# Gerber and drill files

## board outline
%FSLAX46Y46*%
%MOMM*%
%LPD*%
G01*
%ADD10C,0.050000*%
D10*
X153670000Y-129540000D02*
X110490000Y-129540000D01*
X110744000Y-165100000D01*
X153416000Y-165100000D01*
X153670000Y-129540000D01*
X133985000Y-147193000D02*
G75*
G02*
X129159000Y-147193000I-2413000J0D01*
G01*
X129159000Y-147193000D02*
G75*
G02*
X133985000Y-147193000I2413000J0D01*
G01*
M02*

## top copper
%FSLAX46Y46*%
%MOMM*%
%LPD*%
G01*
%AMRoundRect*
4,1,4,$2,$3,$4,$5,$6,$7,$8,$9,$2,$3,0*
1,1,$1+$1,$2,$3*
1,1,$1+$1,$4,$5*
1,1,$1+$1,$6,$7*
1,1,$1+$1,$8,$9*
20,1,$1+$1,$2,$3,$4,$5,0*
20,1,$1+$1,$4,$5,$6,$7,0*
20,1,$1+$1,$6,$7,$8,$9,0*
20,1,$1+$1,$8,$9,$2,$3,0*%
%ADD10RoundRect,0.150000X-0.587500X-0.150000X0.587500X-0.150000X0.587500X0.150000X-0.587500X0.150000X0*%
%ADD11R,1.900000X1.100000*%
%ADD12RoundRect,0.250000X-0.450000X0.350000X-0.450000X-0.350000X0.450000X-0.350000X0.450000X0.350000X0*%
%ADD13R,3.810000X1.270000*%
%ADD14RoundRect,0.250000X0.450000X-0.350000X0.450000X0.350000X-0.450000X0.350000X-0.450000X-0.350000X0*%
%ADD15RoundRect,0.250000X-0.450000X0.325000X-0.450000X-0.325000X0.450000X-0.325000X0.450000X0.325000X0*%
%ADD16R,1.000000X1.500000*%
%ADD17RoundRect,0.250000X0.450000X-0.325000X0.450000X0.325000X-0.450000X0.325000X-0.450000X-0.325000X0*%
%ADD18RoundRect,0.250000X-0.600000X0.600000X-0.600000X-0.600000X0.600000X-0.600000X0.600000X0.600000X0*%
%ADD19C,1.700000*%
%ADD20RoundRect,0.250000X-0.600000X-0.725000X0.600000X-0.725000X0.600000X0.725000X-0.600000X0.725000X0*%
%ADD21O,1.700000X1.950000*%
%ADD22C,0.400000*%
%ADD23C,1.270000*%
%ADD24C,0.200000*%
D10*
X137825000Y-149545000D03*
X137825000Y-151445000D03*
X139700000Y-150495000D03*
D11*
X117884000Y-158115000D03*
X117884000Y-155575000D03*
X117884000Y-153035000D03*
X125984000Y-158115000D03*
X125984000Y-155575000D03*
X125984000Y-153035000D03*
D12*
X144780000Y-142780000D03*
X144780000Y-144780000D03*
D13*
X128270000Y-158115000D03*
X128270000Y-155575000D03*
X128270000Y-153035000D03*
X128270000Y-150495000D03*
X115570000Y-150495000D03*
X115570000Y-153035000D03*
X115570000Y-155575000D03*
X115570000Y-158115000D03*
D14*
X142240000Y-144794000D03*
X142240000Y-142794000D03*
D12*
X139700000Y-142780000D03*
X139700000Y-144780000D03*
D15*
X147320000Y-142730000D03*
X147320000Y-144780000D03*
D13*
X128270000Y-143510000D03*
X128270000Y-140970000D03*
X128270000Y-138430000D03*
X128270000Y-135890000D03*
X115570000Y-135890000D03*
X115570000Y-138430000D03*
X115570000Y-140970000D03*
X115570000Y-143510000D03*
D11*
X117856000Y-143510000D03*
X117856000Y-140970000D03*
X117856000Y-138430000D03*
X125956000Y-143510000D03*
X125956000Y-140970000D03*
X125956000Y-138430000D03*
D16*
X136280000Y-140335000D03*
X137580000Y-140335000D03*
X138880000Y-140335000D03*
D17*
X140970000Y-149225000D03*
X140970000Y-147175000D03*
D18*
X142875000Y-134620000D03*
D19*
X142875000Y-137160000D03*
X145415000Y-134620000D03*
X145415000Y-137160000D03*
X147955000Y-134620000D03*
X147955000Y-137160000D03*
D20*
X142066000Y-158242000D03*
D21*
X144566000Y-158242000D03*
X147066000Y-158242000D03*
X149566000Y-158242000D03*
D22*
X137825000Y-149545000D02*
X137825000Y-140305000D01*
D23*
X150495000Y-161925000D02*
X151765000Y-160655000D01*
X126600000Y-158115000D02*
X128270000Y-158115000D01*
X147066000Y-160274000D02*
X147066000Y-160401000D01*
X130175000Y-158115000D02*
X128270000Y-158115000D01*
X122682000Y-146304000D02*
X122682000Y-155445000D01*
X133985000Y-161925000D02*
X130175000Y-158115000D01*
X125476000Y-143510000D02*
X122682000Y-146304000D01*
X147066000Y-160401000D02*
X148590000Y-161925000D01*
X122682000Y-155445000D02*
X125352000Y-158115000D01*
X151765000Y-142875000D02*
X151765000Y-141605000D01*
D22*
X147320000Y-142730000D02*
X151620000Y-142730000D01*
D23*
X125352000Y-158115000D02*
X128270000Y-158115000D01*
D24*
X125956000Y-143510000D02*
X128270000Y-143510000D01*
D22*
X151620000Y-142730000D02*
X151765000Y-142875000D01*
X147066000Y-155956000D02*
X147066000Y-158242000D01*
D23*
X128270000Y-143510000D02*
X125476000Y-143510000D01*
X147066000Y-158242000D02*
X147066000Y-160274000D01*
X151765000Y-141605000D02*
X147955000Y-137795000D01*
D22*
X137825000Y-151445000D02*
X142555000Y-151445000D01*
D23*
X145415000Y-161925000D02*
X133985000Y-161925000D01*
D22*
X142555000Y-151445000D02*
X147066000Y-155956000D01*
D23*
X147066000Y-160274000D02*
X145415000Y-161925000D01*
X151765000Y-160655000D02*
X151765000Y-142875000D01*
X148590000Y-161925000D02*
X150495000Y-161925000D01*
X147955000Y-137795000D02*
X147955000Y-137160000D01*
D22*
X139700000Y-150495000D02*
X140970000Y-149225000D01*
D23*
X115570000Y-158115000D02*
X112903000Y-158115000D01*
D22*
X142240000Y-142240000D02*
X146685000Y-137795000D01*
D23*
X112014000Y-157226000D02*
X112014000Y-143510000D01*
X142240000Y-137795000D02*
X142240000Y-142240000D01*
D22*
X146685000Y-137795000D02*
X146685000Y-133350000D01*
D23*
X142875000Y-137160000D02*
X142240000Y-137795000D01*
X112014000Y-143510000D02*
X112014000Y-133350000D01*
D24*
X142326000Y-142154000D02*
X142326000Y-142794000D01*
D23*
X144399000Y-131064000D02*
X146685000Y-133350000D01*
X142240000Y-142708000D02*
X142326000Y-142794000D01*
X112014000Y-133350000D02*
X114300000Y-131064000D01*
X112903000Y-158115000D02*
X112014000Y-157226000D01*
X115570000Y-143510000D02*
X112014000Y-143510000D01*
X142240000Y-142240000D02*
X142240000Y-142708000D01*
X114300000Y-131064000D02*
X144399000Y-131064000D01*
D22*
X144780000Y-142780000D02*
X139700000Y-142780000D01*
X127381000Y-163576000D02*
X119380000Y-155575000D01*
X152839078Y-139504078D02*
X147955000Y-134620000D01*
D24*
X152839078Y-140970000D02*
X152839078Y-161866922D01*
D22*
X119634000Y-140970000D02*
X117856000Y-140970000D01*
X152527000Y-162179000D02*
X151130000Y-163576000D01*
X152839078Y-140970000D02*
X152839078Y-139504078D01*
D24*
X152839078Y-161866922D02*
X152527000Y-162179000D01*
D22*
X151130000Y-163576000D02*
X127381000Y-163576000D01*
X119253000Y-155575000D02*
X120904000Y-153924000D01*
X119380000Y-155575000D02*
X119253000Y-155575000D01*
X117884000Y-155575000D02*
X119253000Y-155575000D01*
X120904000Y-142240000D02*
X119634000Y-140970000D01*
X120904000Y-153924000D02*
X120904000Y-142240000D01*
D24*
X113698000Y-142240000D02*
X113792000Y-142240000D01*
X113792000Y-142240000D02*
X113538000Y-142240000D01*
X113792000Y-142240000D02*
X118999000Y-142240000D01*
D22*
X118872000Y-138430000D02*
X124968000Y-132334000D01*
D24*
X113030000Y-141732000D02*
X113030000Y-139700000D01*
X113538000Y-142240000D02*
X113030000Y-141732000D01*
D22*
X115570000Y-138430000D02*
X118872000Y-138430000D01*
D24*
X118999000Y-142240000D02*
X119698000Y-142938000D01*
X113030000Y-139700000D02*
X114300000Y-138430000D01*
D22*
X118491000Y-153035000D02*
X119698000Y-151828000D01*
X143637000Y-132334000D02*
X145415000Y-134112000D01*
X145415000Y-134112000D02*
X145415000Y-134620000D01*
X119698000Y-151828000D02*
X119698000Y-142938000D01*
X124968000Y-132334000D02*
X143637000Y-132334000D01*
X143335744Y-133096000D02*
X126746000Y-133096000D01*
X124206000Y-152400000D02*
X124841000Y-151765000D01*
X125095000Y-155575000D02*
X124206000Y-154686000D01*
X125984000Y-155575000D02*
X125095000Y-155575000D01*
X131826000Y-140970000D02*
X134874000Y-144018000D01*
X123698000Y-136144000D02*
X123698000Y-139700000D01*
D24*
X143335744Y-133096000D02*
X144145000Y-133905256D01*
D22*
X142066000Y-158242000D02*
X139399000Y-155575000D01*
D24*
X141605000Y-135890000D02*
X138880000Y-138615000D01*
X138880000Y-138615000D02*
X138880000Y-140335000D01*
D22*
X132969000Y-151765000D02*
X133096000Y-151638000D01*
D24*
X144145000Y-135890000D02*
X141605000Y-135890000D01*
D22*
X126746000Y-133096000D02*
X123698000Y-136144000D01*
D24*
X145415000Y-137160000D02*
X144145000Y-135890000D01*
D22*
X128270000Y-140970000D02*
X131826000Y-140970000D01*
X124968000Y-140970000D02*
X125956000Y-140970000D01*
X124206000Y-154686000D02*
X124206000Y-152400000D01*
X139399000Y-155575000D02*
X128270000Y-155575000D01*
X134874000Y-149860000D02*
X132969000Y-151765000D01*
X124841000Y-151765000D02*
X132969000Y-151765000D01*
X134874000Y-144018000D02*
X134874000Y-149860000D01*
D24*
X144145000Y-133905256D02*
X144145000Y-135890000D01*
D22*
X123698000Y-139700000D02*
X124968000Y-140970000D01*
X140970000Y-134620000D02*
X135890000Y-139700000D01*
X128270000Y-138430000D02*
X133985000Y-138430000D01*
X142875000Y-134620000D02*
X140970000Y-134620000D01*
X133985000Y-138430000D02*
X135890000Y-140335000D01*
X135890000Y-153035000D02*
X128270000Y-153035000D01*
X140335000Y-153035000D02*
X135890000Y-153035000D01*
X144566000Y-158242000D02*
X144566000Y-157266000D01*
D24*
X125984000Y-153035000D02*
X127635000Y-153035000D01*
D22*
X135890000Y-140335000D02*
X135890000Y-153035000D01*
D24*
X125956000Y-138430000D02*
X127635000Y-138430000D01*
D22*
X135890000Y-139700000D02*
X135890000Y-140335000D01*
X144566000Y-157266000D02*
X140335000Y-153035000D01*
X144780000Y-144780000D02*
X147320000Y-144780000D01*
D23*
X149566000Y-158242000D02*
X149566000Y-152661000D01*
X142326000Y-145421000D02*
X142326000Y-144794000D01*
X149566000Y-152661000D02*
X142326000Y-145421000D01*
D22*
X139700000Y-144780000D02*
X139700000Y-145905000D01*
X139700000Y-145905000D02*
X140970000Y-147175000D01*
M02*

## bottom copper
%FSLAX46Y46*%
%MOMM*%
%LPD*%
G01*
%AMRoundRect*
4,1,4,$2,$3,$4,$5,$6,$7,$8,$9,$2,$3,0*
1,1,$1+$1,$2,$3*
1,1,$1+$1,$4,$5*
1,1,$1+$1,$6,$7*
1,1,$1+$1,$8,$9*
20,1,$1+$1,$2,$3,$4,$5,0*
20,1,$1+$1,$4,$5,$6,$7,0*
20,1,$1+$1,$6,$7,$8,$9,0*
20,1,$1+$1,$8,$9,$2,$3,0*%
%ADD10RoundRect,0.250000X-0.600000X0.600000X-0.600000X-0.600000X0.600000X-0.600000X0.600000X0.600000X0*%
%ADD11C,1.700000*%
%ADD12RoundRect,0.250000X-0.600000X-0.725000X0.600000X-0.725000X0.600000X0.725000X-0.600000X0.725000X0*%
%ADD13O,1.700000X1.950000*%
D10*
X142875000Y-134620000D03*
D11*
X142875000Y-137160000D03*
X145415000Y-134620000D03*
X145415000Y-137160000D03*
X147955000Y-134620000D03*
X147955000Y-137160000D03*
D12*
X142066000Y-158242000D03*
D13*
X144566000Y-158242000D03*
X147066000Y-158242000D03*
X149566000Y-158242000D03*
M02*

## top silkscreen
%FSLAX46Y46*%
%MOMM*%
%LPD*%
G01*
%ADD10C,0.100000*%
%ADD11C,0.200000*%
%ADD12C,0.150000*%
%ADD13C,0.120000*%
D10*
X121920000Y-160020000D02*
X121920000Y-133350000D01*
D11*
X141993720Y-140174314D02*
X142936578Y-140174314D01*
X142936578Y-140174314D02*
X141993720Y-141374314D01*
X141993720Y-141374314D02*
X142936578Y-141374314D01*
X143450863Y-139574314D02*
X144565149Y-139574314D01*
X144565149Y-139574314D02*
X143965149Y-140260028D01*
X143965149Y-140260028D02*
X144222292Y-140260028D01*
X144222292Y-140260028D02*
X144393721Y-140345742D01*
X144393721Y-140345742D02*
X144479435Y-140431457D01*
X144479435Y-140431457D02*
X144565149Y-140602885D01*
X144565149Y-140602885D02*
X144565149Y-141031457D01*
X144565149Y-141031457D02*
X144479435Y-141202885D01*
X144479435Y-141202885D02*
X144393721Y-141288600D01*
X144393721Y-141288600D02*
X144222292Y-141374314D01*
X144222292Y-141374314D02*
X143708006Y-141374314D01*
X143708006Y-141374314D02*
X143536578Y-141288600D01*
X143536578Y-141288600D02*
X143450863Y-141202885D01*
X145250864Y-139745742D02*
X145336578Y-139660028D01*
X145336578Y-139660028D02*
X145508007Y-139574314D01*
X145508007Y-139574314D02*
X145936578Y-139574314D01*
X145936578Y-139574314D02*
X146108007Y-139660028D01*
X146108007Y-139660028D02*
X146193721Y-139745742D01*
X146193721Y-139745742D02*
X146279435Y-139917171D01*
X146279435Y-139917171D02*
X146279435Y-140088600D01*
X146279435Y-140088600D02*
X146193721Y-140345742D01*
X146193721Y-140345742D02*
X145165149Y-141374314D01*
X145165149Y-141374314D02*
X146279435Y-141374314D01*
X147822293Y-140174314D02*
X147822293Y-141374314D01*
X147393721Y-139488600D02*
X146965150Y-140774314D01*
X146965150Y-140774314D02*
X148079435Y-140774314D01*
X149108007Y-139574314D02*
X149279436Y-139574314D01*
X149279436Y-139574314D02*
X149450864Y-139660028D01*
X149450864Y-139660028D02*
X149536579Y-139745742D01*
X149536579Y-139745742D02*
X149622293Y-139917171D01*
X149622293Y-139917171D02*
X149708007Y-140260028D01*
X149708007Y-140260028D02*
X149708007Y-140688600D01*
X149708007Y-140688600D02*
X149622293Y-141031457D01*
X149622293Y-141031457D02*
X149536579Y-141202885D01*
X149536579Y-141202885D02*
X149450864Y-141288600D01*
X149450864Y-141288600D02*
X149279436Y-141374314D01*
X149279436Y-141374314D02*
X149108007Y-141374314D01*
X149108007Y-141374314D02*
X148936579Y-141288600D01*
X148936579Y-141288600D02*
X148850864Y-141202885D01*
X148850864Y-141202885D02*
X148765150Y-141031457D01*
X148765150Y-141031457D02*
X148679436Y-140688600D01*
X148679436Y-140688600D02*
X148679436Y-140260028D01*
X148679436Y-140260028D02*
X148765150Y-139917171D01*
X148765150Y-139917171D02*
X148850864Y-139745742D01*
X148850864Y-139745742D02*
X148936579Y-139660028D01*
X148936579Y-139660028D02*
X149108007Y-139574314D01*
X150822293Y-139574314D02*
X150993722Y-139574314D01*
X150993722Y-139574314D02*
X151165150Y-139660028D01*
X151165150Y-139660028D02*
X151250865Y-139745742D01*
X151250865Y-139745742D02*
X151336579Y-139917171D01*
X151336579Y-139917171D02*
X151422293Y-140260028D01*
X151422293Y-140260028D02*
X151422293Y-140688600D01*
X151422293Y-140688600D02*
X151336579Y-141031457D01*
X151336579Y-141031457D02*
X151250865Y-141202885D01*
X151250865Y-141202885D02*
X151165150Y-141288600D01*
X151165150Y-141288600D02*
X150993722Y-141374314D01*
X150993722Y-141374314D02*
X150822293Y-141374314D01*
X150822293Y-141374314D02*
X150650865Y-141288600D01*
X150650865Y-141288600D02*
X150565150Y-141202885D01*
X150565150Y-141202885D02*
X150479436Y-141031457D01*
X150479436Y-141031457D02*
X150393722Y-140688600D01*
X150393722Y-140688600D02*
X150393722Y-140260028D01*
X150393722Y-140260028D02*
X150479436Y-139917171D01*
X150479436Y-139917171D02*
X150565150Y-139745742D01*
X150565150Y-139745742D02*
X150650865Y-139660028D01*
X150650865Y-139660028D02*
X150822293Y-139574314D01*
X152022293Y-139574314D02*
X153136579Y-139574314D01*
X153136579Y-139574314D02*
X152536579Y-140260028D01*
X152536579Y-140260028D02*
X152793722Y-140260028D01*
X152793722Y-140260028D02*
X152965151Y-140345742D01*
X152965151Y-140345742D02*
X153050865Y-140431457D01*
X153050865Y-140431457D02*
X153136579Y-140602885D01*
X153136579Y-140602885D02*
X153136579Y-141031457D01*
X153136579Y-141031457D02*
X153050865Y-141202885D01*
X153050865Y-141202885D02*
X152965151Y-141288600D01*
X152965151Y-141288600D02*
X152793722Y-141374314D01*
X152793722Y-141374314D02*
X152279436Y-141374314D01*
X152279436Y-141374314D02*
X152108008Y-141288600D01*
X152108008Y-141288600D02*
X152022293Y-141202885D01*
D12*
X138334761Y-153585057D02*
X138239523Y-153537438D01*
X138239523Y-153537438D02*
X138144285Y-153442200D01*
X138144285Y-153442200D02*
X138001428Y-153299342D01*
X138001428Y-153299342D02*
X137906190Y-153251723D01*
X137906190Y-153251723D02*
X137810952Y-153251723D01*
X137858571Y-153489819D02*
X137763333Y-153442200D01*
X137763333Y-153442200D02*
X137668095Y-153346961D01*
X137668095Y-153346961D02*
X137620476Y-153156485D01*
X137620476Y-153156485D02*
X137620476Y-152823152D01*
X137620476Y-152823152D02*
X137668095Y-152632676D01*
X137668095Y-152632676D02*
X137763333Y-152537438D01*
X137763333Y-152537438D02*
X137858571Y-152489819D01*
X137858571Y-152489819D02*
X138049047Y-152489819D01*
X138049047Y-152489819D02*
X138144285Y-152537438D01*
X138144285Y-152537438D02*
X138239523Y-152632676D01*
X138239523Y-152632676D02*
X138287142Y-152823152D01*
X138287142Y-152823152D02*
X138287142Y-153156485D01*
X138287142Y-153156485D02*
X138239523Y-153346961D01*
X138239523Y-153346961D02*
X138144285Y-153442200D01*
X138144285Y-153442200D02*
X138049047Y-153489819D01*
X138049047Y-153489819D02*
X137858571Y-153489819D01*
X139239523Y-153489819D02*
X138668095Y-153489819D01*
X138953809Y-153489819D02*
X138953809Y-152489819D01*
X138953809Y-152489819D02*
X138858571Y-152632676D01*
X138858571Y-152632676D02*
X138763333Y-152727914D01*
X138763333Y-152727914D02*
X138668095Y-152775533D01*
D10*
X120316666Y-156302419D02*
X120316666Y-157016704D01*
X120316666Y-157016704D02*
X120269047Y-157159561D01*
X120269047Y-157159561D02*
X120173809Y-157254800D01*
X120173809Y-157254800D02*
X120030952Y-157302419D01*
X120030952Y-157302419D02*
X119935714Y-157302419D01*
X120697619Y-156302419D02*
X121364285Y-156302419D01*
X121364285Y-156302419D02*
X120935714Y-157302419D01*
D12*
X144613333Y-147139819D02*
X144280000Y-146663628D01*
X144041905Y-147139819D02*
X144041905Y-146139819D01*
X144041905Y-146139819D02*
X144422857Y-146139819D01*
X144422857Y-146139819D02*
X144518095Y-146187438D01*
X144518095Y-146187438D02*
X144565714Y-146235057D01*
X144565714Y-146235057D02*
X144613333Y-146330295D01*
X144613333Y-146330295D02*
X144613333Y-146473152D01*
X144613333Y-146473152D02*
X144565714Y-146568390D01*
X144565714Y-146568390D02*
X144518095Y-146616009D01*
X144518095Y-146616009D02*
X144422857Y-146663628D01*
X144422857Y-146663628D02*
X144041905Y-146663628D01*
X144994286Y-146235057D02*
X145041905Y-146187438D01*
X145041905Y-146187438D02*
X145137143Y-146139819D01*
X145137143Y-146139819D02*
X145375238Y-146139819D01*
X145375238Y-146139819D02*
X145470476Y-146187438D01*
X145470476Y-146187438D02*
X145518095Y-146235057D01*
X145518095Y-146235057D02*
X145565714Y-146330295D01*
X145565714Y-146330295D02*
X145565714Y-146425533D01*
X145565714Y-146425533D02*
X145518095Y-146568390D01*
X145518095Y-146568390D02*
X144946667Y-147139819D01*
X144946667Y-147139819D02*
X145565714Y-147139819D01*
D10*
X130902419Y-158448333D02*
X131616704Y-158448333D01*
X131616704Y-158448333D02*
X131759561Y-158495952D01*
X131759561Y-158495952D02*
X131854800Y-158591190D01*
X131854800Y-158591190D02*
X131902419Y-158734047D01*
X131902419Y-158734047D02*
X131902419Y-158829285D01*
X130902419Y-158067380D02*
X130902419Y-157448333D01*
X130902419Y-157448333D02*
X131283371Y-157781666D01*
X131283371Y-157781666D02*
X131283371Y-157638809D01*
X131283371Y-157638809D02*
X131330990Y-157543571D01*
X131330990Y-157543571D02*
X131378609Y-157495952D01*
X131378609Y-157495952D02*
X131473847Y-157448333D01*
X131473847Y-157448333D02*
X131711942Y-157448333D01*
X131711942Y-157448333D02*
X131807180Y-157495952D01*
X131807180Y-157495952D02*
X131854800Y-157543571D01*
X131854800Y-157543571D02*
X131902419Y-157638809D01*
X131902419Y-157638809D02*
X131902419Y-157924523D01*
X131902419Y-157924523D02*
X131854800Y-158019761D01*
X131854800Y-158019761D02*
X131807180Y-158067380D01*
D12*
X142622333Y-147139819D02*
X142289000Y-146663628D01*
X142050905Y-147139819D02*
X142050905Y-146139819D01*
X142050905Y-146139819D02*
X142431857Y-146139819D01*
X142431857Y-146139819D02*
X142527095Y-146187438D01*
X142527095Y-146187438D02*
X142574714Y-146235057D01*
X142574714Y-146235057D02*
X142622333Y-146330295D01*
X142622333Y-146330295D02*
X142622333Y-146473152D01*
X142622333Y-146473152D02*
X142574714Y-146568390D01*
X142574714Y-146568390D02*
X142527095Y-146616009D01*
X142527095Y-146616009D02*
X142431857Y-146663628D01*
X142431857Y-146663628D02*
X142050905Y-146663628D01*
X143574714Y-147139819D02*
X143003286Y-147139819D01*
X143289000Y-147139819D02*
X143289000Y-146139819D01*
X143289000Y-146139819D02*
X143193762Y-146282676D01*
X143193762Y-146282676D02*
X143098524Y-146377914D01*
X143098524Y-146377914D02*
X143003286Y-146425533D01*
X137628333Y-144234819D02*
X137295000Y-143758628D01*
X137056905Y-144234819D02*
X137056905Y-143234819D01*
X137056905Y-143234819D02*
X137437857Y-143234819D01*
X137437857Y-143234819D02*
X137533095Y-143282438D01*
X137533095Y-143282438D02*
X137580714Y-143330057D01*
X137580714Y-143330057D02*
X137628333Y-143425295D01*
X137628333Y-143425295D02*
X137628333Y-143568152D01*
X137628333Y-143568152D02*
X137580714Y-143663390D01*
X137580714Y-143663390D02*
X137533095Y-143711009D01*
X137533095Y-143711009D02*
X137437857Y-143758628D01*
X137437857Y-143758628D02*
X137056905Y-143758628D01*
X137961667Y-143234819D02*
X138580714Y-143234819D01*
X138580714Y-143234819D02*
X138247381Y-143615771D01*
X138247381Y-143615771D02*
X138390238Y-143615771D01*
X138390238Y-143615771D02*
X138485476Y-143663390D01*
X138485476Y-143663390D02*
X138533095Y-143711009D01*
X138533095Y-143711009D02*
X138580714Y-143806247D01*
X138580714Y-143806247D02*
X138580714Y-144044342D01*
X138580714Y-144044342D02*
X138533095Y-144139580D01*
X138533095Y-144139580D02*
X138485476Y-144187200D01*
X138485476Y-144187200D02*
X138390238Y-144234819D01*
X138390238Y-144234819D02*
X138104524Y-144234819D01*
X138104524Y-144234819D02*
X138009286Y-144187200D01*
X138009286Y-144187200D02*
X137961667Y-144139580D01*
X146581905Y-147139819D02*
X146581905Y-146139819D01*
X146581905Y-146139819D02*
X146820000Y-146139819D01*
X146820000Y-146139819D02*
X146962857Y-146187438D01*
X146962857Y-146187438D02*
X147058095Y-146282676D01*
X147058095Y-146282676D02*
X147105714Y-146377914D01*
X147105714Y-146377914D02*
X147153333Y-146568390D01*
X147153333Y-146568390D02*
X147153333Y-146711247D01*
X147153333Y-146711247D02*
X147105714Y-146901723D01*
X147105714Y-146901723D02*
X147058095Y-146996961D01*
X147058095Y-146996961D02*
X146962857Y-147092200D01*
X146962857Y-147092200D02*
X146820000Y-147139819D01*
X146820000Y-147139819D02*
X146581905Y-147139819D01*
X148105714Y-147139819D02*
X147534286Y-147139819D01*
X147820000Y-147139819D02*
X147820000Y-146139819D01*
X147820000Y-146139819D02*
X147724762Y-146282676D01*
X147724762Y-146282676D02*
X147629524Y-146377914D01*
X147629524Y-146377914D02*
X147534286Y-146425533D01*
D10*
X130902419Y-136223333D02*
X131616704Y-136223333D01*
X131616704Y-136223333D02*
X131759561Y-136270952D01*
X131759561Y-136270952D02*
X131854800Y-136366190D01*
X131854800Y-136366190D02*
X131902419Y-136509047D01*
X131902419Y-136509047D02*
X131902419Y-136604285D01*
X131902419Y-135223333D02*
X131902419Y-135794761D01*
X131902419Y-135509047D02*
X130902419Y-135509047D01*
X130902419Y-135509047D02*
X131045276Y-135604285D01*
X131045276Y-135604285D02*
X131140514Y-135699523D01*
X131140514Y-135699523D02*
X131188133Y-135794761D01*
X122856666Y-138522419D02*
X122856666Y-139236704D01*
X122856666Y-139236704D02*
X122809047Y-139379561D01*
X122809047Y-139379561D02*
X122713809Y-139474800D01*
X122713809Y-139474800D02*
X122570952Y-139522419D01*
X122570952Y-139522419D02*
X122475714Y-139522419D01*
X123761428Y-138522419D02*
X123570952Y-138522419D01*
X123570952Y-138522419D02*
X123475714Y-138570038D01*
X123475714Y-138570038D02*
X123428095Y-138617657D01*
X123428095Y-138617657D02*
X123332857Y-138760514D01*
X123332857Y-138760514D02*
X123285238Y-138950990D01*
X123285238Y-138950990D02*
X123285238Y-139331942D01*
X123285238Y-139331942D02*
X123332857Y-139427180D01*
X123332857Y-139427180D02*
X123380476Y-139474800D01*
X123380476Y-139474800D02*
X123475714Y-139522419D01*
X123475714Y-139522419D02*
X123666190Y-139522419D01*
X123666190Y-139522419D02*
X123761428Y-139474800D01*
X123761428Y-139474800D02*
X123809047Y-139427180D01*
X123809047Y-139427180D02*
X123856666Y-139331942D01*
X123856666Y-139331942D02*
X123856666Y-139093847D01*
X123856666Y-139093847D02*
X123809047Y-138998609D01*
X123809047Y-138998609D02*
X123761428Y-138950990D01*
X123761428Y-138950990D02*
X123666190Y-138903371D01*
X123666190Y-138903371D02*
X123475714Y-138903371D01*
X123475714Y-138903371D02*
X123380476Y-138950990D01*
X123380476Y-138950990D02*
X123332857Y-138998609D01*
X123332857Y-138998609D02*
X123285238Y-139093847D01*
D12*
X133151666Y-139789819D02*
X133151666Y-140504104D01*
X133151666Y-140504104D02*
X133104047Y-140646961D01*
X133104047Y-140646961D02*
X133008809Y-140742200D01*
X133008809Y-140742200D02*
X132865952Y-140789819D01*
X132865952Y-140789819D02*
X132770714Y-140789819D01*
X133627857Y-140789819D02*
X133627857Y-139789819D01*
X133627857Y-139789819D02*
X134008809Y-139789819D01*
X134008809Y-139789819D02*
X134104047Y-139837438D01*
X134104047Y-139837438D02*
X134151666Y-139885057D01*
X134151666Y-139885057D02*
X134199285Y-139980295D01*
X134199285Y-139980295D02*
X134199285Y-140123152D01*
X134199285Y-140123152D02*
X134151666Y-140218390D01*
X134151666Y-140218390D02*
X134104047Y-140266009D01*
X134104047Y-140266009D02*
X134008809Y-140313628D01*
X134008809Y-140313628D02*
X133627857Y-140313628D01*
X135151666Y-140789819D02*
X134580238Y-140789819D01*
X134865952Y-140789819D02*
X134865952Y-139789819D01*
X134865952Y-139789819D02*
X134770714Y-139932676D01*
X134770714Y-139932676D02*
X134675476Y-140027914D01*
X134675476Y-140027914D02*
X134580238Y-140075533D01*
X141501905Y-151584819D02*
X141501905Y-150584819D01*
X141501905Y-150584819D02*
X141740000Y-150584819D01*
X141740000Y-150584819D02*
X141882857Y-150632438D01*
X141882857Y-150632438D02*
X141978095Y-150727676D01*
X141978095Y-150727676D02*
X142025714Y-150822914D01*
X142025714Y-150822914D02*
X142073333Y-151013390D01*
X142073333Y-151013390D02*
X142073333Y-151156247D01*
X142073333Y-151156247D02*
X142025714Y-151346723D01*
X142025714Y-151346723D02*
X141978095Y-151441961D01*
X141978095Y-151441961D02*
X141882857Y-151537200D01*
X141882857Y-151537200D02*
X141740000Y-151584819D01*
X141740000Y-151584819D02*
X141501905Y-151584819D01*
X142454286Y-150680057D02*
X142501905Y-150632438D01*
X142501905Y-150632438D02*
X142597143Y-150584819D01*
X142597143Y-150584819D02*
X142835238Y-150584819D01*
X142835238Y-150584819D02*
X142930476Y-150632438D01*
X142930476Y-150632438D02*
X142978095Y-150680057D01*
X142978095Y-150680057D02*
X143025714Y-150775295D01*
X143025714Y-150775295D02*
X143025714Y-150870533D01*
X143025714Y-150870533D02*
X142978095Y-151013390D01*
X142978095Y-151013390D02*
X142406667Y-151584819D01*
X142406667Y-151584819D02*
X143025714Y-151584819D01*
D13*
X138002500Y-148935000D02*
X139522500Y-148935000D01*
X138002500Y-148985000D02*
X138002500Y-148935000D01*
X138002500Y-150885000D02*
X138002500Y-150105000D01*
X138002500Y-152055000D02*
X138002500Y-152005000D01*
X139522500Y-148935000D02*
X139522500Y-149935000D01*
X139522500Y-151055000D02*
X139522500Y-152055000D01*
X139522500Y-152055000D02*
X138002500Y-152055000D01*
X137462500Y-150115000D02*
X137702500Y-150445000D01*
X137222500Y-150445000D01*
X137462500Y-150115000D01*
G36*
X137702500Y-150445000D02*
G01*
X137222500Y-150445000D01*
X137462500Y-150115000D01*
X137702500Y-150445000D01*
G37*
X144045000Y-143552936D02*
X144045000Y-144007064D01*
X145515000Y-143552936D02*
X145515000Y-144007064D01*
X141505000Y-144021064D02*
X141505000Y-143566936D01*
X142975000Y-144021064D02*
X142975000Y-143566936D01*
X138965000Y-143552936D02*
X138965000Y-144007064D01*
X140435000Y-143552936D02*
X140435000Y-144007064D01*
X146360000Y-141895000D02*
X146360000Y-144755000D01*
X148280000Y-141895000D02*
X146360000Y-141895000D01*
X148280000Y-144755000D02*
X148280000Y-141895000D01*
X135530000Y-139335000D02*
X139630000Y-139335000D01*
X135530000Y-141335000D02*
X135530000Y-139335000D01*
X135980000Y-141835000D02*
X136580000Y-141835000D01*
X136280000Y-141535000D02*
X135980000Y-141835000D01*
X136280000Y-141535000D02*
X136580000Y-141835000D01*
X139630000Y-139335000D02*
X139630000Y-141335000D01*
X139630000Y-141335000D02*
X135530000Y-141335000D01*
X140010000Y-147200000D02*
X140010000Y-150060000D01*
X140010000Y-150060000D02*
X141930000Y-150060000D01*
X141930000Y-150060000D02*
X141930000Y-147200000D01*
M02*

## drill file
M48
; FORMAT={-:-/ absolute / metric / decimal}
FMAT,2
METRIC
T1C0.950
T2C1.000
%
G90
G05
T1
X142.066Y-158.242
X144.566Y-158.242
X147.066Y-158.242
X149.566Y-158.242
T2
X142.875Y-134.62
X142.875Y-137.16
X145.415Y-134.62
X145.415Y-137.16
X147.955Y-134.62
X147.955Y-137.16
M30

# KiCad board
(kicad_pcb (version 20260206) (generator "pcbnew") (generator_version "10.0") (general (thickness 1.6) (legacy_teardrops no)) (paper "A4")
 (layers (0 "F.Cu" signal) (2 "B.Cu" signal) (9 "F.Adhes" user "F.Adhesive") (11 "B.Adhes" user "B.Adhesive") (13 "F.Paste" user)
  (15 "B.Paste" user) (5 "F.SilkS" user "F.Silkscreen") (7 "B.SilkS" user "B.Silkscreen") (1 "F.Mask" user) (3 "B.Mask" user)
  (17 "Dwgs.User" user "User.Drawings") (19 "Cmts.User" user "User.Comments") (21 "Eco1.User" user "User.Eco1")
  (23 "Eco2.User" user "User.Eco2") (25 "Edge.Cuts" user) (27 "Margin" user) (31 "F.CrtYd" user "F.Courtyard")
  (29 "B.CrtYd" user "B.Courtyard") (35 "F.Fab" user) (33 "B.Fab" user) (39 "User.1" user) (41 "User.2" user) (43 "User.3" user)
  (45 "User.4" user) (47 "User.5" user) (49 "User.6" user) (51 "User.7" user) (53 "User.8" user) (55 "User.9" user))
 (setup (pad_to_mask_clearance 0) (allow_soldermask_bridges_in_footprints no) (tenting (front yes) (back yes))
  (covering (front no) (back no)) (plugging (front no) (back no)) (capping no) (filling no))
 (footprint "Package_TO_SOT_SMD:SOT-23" (layer "F.Cu") (at 138.7625 150.495)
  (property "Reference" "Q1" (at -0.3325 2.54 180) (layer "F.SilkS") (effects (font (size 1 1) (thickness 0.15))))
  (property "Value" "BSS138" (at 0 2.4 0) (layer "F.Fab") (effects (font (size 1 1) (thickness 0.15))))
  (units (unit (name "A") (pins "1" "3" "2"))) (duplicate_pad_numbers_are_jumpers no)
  (fp_line (start -0.76 -1.56) (end 0.76 -1.56) (stroke (width 0.12) (type solid)) (layer "F.SilkS"))
  (fp_line (start -0.76 -1.51) (end -0.76 -1.56) (stroke (width 0.12) (type solid)) (layer "F.SilkS"))
  (fp_line (start -0.76 0.39) (end -0.76 -0.39) (stroke (width 0.12) (type solid)) (layer "F.SilkS"))
  (fp_line (start -0.76 1.56) (end -0.76 1.51) (stroke (width 0.12) (type solid)) (layer "F.SilkS"))
  (fp_line (start 0.76 -1.56) (end 0.76 -0.56) (stroke (width 0.12) (type solid)) (layer "F.SilkS"))
  (fp_line (start 0.76 0.56) (end 0.76 1.56) (stroke (width 0.12) (type solid)) (layer "F.SilkS"))
  (fp_line (start 0.76 1.56) (end -0.76 1.56) (stroke (width 0.12) (type solid)) (layer "F.SilkS"))
  (fp_poly (pts (xy -1.3 -0.38) (xy -1.06 -0.05) (xy -1.54 -0.05)) (stroke (width 0.12) (type solid)) (fill yes) (layer "F.SilkS"))
  (pad "1" smd roundrect (at -0.9375 -0.95) (size 1.475 0.6) (layers "F.Cu" "F.Mask" "F.Paste") (roundrect_rratio 0.25) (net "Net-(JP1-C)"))
  (pad "2" smd roundrect (at -0.9375 0.95) (size 1.475 0.6) (layers "F.Cu" "F.Mask" "F.Paste") (roundrect_rratio 0.25) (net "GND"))
  (pad "3" smd roundrect (at 0.9375 0) (size 1.475 0.6) (layers "F.Cu" "F.Mask" "F.Paste") (roundrect_rratio 0.25) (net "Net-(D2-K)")))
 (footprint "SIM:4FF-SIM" (layer "F.Cu") (at 121.934 149.225)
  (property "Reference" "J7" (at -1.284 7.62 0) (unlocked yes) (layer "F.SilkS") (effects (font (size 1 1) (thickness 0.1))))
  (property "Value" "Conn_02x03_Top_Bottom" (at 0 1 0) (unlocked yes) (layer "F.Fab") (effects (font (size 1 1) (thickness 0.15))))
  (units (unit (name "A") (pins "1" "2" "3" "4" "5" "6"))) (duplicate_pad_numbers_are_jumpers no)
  (pad "1" smd rect (at -4.05 8.89) (size 1.9 1.1) (layers "F.Cu" "F.Mask" "F.Paste") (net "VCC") (thermal_bridge_angle 45))
  (pad "2" smd rect (at -4.05 6.35) (size 1.9 1.1) (layers "F.Cu" "F.Mask" "F.Paste") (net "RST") (thermal_bridge_angle 45))
  (pad "3" smd rect (at -4.05 3.81) (size 1.9 1.1) (layers "F.Cu" "F.Mask" "F.Paste") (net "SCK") (thermal_bridge_angle 45))
  (pad "4" smd rect (at 4.05 8.89) (size 1.9 1.1) (layers "F.Cu" "F.Mask" "F.Paste") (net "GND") (thermal_bridge_angle 45))
  (pad "5" smd rect (at 4.05 6.35) (size 1.9 1.1) (layers "F.Cu" "F.Mask" "F.Paste") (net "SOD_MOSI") (thermal_bridge_angle 45))
  (pad "6" smd rect (at 4.05 3.81) (size 1.9 1.1) (layers "F.Cu" "F.Mask" "F.Paste") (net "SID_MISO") (thermal_bridge_angle 45)))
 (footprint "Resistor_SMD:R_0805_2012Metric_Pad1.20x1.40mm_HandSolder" (layer "F.Cu") (at 144.78 143.78 -90)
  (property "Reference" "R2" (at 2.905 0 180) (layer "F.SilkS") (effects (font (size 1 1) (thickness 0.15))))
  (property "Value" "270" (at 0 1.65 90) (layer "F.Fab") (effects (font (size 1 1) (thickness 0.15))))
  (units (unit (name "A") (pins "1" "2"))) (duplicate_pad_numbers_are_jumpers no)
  (fp_line (start -0.227064 0.735) (end 0.227064 0.735) (stroke (width 0.12) (type solid)) (layer "F.SilkS"))
  (fp_line (start -0.227064 -0.735) (end 0.227064 -0.735) (stroke (width 0.12) (type solid)) (layer "F.SilkS"))
  (pad "1" smd roundrect (at -1 0 270) (size 1.2 1.4) (layers "F.Cu" "F.Mask" "F.Paste") (roundrect_rratio 0.208333) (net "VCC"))
  (pad "2" smd roundrect (at 1 0 270) (size 1.2 1.4) (layers "F.Cu" "F.Mask" "F.Paste") (roundrect_rratio 0.208333) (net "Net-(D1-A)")))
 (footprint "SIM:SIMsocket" (layer "F.Cu") (at 112.395 153.035 90)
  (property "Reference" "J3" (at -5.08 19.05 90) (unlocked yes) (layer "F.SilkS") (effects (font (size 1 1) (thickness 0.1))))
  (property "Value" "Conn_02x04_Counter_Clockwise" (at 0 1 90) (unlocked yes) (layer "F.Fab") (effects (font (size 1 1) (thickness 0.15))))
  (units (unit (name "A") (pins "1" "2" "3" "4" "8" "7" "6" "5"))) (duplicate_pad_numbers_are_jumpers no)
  (pad "1" smd rect (at -5.08 15.875 90) (size 1.27 3.81) (layers "F.Cu" "F.Mask") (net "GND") (thermal_bridge_angle 45))
  (pad "2" smd rect (at -2.54 15.875 90) (size 1.27 3.81) (layers "F.Cu" "F.Mask") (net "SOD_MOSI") (thermal_bridge_angle 45))
  (pad "3" smd rect (at 0 15.875 90) (size 1.27 3.81) (layers "F.Cu" "F.Mask") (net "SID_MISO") (thermal_bridge_angle 45))
  (pad "4" smd rect (at 2.54 15.875 90) (size 1.27 3.81) (layers "F.Cu" "F.Mask") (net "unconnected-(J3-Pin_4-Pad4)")
   (thermal_bridge_angle 45))
  (pad "5" smd rect (at 2.54 3.175 90) (size 1.27 3.81) (layers "F.Cu" "F.Mask") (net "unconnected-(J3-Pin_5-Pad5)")
   (thermal_bridge_angle 45))
  (pad "6" smd rect (at 0 3.175 90) (size 1.27 3.81) (layers "F.Cu" "F.Mask") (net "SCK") (thermal_bridge_angle 45))
  (pad "7" smd rect (at -2.54 3.175 90) (size 1.27 3.81) (layers "F.Cu" "F.Mask") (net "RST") (thermal_bridge_angle 45))
  (pad "8" smd rect (at -5.08 3.175 90) (size 1.27 3.81) (layers "F.Cu" "F.Mask") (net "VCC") (thermal_bridge_angle 45)))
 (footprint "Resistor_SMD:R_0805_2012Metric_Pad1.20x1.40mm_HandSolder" (layer "F.Cu") (at 142.24 143.794 90)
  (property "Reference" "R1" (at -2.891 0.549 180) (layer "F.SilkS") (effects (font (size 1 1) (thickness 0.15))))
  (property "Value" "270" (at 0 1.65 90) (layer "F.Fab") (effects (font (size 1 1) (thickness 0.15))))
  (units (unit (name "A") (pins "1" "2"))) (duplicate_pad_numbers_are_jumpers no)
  (fp_line (start -0.227064 -0.735) (end 0.227064 -0.735) (stroke (width 0.12) (type solid)) (layer "F.SilkS"))
  (fp_line (start -0.227064 0.735) (end 0.227064 0.735) (stroke (width 0.12) (type solid)) (layer "F.SilkS"))
  (pad "1" smd roundrect (at -1 0 90) (size 1.2 1.4) (layers "F.Cu" "F.Mask" "F.Paste") (roundrect_rratio 0.208333) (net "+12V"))
  (pad "2" smd roundrect (at 1 0 90) (size 1.2 1.4) (layers "F.Cu" "F.Mask" "F.Paste") (roundrect_rratio 0.208333) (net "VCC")))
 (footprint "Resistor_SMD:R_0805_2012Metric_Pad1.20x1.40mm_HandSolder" (layer "F.Cu") (at 139.7 143.78 -90)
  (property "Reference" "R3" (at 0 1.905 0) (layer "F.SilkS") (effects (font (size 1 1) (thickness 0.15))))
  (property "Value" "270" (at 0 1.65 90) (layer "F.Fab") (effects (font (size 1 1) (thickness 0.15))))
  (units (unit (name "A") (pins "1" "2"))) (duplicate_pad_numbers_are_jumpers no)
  (fp_line (start -0.227064 0.735) (end 0.227064 0.735) (stroke (width 0.12) (type solid)) (layer "F.SilkS"))
  (fp_line (start -0.227064 -0.735) (end 0.227064 -0.735) (stroke (width 0.12) (type solid)) (layer "F.SilkS"))
  (pad "1" smd roundrect (at -1 0 270) (size 1.2 1.4) (layers "F.Cu" "F.Mask" "F.Paste") (roundrect_rratio 0.208333) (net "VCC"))
  (pad "2" smd roundrect (at 1 0 270) (size 1.2 1.4) (layers "F.Cu" "F.Mask" "F.Paste") (roundrect_rratio 0.208333) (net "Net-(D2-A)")))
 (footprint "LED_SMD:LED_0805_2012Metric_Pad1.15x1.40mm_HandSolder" (layer "F.Cu") (at 147.32 143.755 -90)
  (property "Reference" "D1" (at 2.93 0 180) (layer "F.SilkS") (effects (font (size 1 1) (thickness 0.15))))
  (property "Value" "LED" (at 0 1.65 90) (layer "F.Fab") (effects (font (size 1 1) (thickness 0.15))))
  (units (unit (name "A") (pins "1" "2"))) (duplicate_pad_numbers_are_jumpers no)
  (fp_line (start -1.86 0.96) (end 1 0.96) (stroke (width 0.12) (type solid)) (layer "F.SilkS"))
  (fp_line (start -1.86 -0.96) (end -1.86 0.96) (stroke (width 0.12) (type solid)) (layer "F.SilkS"))
  (fp_line (start 1 -0.96) (end -1.86 -0.96) (stroke (width 0.12) (type solid)) (layer "F.SilkS"))
  (pad "1" smd roundrect (at -1.025 0 270) (size 1.15 1.4) (layers "F.Cu" "F.Mask" "F.Paste") (roundrect_rratio 0.217391) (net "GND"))
  (pad "2" smd roundrect (at 1.025 0 270) (size 1.15 1.4) (layers "F.Cu" "F.Mask" "F.Paste") (roundrect_rratio 0.217391) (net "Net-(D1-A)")))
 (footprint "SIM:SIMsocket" (layer "F.Cu") (at 112.395 138.43 90)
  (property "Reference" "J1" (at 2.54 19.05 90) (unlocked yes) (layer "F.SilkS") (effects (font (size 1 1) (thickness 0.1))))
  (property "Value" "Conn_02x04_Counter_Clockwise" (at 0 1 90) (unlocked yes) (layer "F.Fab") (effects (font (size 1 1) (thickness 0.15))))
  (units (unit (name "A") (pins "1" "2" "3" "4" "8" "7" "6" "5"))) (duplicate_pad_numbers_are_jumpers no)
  (pad "1" smd rect (at -5.08 15.875 90) (size 1.27 3.81) (layers "F.Cu" "F.Mask") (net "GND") (thermal_bridge_angle 45))
  (pad "2" smd rect (at -2.54 15.875 90) (size 1.27 3.81) (layers "F.Cu" "F.Mask") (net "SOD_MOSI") (thermal_bridge_angle 45))
  (pad "3" smd rect (at 0 15.875 90) (size 1.27 3.81) (layers "F.Cu" "F.Mask") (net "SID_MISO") (thermal_bridge_angle 45))
  (pad "4" smd rect (at 2.54 15.875 90) (size 1.27 3.81) (layers "F.Cu" "F.Mask") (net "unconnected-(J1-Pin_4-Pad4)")
   (thermal_bridge_angle 45))
  (pad "5" smd rect (at 2.54 3.175 90) (size 1.27 3.81) (layers "F.Cu" "F.Mask") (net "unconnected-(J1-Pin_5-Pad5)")
   (thermal_bridge_angle 45))
  (pad "6" smd rect (at 0 3.175 90) (size 1.27 3.81) (layers "F.Cu" "F.Mask") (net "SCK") (thermal_bridge_angle 45))
  (pad "7" smd rect (at -2.54 3.175 90) (size 1.27 3.81) (layers "F.Cu" "F.Mask") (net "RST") (thermal_bridge_angle 45))
  (pad "8" smd rect (at -5.08 3.175 90) (size 1.27 3.81) (layers "F.Cu" "F.Mask") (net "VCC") (thermal_bridge_angle 45)))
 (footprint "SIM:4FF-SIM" (layer "F.Cu") (at 121.906 134.62)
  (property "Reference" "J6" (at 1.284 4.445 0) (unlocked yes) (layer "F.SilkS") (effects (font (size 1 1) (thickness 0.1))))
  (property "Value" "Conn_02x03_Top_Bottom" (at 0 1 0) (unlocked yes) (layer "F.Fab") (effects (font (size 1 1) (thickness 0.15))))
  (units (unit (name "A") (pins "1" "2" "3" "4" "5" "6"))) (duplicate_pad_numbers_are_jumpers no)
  (pad "1" smd rect (at -4.05 8.89) (size 1.9 1.1) (layers "F.Cu" "F.Mask" "F.Paste") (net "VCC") (thermal_bridge_angle 45))
  (pad "2" smd rect (at -4.05 6.35) (size 1.9 1.1) (layers "F.Cu" "F.Mask" "F.Paste") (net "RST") (thermal_bridge_angle 45))
  (pad "3" smd rect (at -4.05 3.81) (size 1.9 1.1) (layers "F.Cu" "F.Mask" "F.Paste") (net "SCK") (thermal_bridge_angle 45))
  (pad "4" smd rect (at 4.05 8.89) (size 1.9 1.1) (layers "F.Cu" "F.Mask" "F.Paste") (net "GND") (thermal_bridge_angle 45))
  (pad "5" smd rect (at 4.05 6.35) (size 1.9 1.1) (layers "F.Cu" "F.Mask" "F.Paste") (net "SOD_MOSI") (thermal_bridge_angle 45))
  (pad "6" smd rect (at 4.05 3.81) (size 1.9 1.1) (layers "F.Cu" "F.Mask" "F.Paste") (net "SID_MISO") (thermal_bridge_angle 45)))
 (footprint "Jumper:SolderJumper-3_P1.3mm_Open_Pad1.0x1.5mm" (layer "F.Cu") (at 137.58 140.335)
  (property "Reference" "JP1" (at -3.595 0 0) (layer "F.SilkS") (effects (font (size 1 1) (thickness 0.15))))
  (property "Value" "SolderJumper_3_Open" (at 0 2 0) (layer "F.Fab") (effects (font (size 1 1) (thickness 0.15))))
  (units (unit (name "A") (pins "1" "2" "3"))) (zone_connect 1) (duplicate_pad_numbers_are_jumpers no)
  (fp_line (start -2.05 -1) (end 2.05 -1) (stroke (width 0.12) (type solid)) (layer "F.SilkS"))
  (fp_line (start -2.05 1) (end -2.05 -1) (stroke (width 0.12) (type solid)) (layer "F.SilkS"))
  (fp_line (start -1.6 1.5) (end -1 1.5) (stroke (width 0.12) (type solid)) (layer "F.SilkS"))
  (fp_line (start -1.3 1.2) (end -1.6 1.5) (stroke (width 0.12) (type solid)) (layer "F.SilkS"))
  (fp_line (start -1.3 1.2) (end -1 1.5) (stroke (width 0.12) (type solid)) (layer "F.SilkS"))
  (fp_line (start 2.05 -1) (end 2.05 1) (stroke (width 0.12) (type solid)) (layer "F.SilkS"))
  (fp_line (start 2.05 1) (end -2.05 1) (stroke (width 0.12) (type solid)) (layer "F.SilkS"))
  (pad "1" smd rect (at -1.3 0) (size 1 1.5) (layers "F.Cu" "F.Mask") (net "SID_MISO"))
  (pad "2" smd rect (at 0 0) (size 1 1.5) (layers "F.Cu" "F.Mask") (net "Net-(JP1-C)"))
  (pad "3" smd rect (at 1.3 0) (size 1 1.5) (layers "F.Cu" "F.Mask") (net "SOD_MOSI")))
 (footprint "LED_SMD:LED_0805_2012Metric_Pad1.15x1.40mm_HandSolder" (layer "F.Cu") (at 140.97 148.2 90)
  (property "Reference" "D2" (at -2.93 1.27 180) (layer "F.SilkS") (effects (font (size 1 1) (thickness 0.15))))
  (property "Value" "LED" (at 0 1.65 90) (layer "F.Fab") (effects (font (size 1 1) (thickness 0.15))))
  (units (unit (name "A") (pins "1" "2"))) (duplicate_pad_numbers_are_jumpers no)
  (fp_line (start 1 -0.96) (end -1.86 -0.96) (stroke (width 0.12) (type solid)) (layer "F.SilkS"))
  (fp_line (start -1.86 -0.96) (end -1.86 0.96) (stroke (width 0.12) (type solid)) (layer "F.SilkS"))
  (fp_line (start -1.86 0.96) (end 1 0.96) (stroke (width 0.12) (type solid)) (layer "F.SilkS"))
  (pad "1" smd roundrect (at -1.025 0 90) (size 1.15 1.4) (layers "F.Cu" "F.Mask" "F.Paste") (roundrect_rratio 0.217391) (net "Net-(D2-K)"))
  (pad "2" smd roundrect (at 1.025 0 90) (size 1.15 1.4) (layers "F.Cu" "F.Mask" "F.Paste") (roundrect_rratio 0.217391) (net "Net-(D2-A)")))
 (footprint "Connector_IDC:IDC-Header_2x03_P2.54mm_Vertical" (layer "B.Cu") (at 142.875 134.62 -90)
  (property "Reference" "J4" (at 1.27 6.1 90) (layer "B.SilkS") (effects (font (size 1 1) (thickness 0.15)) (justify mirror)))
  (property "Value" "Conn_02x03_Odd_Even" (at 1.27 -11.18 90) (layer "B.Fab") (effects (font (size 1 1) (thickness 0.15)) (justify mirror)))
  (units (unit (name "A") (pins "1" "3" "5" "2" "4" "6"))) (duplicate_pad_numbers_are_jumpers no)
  (pad "1" thru_hole roundrect (at 0 0 270) (size 1.7 1.7) (drill 1) (layers "*.Cu" "*.Mask") (remove_unused_layers no)
   (roundrect_rratio 0.147059) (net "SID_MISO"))
  (pad "2" thru_hole circle (at 2.54 0 270) (size 1.7 1.7) (drill 1) (layers "*.Cu" "*.Mask") (remove_unused_layers no) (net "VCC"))
  (pad "3" thru_hole circle (at 0 -2.54 270) (size 1.7 1.7) (drill 1) (layers "*.Cu" "*.Mask") (remove_unused_layers no) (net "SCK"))
  (pad "4" thru_hole circle (at 2.54 -2.54 270) (size 1.7 1.7) (drill 1) (layers "*.Cu" "*.Mask") (remove_unused_layers no) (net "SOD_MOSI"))
  (pad "5" thru_hole circle (at 0 -5.08 270) (size 1.7 1.7) (drill 1) (layers "*.Cu" "*.Mask") (remove_unused_layers no) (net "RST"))
  (pad "6" thru_hole circle (at 2.54 -5.08 270) (size 1.7 1.7) (drill 1) (layers "*.Cu" "*.Mask") (remove_unused_layers no) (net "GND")))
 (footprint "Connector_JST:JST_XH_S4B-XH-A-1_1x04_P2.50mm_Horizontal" (layer "B.Cu") (at 142.066 158.242)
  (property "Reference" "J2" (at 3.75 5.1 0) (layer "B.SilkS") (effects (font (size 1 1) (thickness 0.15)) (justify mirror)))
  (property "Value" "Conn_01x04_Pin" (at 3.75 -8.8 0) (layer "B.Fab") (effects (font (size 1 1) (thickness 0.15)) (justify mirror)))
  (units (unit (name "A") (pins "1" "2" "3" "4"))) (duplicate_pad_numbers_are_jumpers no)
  (pad "1" thru_hole roundrect (at 0 0) (size 1.7 1.95) (drill 0.95) (layers "*.Cu" "*.Mask") (remove_unused_layers no)
   (roundrect_rratio 0.147059) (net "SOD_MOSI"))
  (pad "2" thru_hole oval (at 2.5 0) (size 1.7 1.95) (drill 0.95) (layers "*.Cu" "*.Mask") (remove_unused_layers no) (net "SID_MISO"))
  (pad "3" thru_hole oval (at 5 0) (size 1.7 1.95) (drill 0.95) (layers "*.Cu" "*.Mask") (remove_unused_layers no) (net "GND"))
  (pad "4" thru_hole oval (at 7.5 0) (size 1.7 1.95) (drill 0.95) (layers "*.Cu" "*.Mask") (remove_unused_layers no) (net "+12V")))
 (gr_line (start 121.92 160.02) (end 121.92 133.35) (stroke (width 0.1) (type default)) (layer "F.SilkS"))
 (gr_poly
  (pts (xy 153.67 129.54) (xy 110.49 129.54) (xy 110.744 165.1) (xy 153.416 165.1)) (stroke (width 0.05) (type solid)) (fill no)
  (layer "Edge.Cuts"))
 (gr_circle (center 131.572 147.193) (end 133.985 147.193) (stroke (width 0.05) (type default)) (fill no) (layer "Edge.Cuts"))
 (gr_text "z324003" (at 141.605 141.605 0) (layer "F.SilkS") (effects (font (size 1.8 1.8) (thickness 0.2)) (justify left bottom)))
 (segment (start 137.825 149.545) (end 137.825 140.305) (width 0.4) (layer "F.Cu") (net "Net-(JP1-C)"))
 (segment (start 150.495 161.925) (end 151.765 160.655) (width 1.27) (layer "F.Cu") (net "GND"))
 (segment (start 126.6 158.115) (end 128.27 158.115) (width 1.27) (layer "F.Cu") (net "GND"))
 (segment (start 147.066 160.274) (end 147.066 160.401) (width 1.27) (layer "F.Cu") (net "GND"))
 (segment (start 130.175 158.115) (end 128.27 158.115) (width 1.27) (layer "F.Cu") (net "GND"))
 (segment (start 122.682 146.304) (end 122.682 155.445) (width 1.27) (layer "F.Cu") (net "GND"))
 (segment (start 133.985 161.925) (end 130.175 158.115) (width 1.27) (layer "F.Cu") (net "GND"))
 (segment (start 125.476 143.51) (end 122.682 146.304) (width 1.27) (layer "F.Cu") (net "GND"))
 (segment (start 147.066 160.401) (end 148.59 161.925) (width 1.27) (layer "F.Cu") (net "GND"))
 (segment (start 122.682 155.445) (end 125.352 158.115) (width 1.27) (layer "F.Cu") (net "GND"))
 (segment (start 151.765 142.875) (end 151.765 141.605) (width 1.27) (layer "F.Cu") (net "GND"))
 (segment (start 147.32 142.73) (end 151.62 142.73) (width 0.4) (layer "F.Cu") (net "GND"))
 (segment (start 125.352 158.115) (end 128.27 158.115) (width 1.27) (layer "F.Cu") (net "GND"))
 (segment (start 125.956 143.51) (end 128.27 143.51) (width 0.2) (layer "F.Cu") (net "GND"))
 (segment (start 151.62 142.73) (end 151.765 142.875) (width 0.4) (layer "F.Cu") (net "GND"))
 (segment (start 147.066 155.956) (end 147.066 158.242) (width 0.4) (layer "F.Cu") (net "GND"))
 (segment (start 128.27 143.51) (end 125.476 143.51) (width 1.27) (layer "F.Cu") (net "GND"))
 (segment (start 147.066 158.242) (end 147.066 160.274) (width 1.27) (layer "F.Cu") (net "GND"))
 (segment (start 151.765 141.605) (end 147.955 137.795) (width 1.27) (layer "F.Cu") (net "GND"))
 (segment (start 137.825 151.445) (end 142.555 151.445) (width 0.4) (layer "F.Cu") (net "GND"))
 (segment (start 145.415 161.925) (end 133.985 161.925) (width 1.27) (layer "F.Cu") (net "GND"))
 (segment (start 142.555 151.445) (end 147.066 155.956) (width 0.4) (layer "F.Cu") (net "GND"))
 (segment (start 147.066 160.274) (end 145.415 161.925) (width 1.27) (layer "F.Cu") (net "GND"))
 (segment (start 151.765 160.655) (end 151.765 142.875) (width 1.27) (layer "F.Cu") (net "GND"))
 (segment (start 148.59 161.925) (end 150.495 161.925) (width 1.27) (layer "F.Cu") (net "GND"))
 (segment (start 147.955 137.795) (end 147.955 137.16) (width 1.27) (layer "F.Cu") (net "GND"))
 (segment (start 139.7 150.495) (end 140.97 149.225) (width 0.4) (layer "F.Cu") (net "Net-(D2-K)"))
 (segment (start 115.57 158.115) (end 112.903 158.115) (width 1.27) (layer "F.Cu") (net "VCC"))
 (segment (start 142.24 142.24) (end 146.685 137.795) (width 0.4) (layer "F.Cu") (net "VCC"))
 (segment (start 112.014 157.226) (end 112.014 143.51) (width 1.27) (layer "F.Cu") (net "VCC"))
 (segment (start 142.24 137.795) (end 142.24 142.24) (width 1.27) (layer "F.Cu") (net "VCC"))
 (segment (start 146.685 137.795) (end 146.685 133.35) (width 0.4) (layer "F.Cu") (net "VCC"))
 (segment (start 142.875 137.16) (end 142.24 137.795) (width 1.27) (layer "F.Cu") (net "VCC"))
 (segment (start 112.014 143.51) (end 112.014 133.35) (width 1.27) (layer "F.Cu") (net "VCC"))
 (segment (start 142.326 142.154) (end 142.326 142.794) (width 0.2) (layer "F.Cu") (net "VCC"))
 (segment (start 144.399 131.064) (end 146.685 133.35) (width 1.27) (layer "F.Cu") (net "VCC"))
 (segment (start 142.24 142.708) (end 142.326 142.794) (width 1.27) (layer "F.Cu") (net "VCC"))
 (segment (start 112.014 133.35) (end 114.3 131.064) (width 1.27) (layer "F.Cu") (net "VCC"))
 (segment (start 112.903 158.115) (end 112.014 157.226) (width 1.27) (layer "F.Cu") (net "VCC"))
 (segment (start 115.57 143.51) (end 112.014 143.51) (width 1.27) (layer "F.Cu") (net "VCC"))
 (segment (start 142.24 142.24) (end 142.24 142.708) (width 1.27) (layer "F.Cu") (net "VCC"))
 (segment (start 114.3 131.064) (end 144.399 131.064) (width 1.27) (layer "F.Cu") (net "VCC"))
 (segment (start 144.78 142.78) (end 139.7 142.78) (width 0.4) (layer "F.Cu") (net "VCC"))
 (segment (start 127.381 163.576) (end 119.38 155.575) (width 0.4) (layer "F.Cu") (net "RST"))
 (segment (start 152.839078 139.504078) (end 147.955 134.62) (width 0.4) (layer "F.Cu") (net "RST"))
 (segment (start 152.839078 140.97) (end 152.839078 161.866922) (width 0.2) (layer "F.Cu") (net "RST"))
 (segment (start 119.634 140.97) (end 117.856 140.97) (width 0.4) (layer "F.Cu") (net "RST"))
 (segment (start 152.527 162.179) (end 151.13 163.576) (width 0.4) (layer "F.Cu") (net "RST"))
 (segment (start 152.839078 140.97) (end 152.839078 139.504078) (width 0.4) (layer "F.Cu") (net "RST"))
 (segment (start 152.839078 161.866922) (end 152.527 162.179) (width 0.2) (layer "F.Cu") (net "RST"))
 (segment (start 151.13 163.576) (end 127.381 163.576) (width 0.4) (layer "F.Cu") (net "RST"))
 (segment (start 119.253 155.575) (end 120.904 153.924) (width 0.4) (layer "F.Cu") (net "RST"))
 (segment (start 119.38 155.575) (end 119.253 155.575) (width 0.4) (layer "F.Cu") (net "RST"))
 (segment (start 117.884 155.575) (end 119.253 155.575) (width 0.4) (layer "F.Cu") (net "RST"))
 (segment (start 120.904 142.24) (end 119.634 140.97) (width 0.4) (layer "F.Cu") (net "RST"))
 (segment (start 120.904 153.924) (end 120.904 142.24) (width 0.4) (layer "F.Cu") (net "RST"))
 (segment (start 113.698 142.24) (end 113.792 142.24) (width 0.2) (layer "F.Cu") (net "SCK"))
 (segment (start 113.792 142.24) (end 113.538 142.24) (width 0.2) (layer "F.Cu") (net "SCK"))
 (segment (start 113.792 142.24) (end 118.999 142.24) (width 0.2) (layer "F.Cu") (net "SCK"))
 (segment (start 118.872 138.43) (end 124.968 132.334) (width 0.4) (layer "F.Cu") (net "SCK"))
 (segment (start 113.03 141.732) (end 113.03 139.7) (width 0.2) (layer "F.Cu") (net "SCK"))
 (segment (start 113.538 142.24) (end 113.03 141.732) (width 0.2) (layer "F.Cu") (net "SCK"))
 (segment (start 115.57 138.43) (end 118.872 138.43) (width 0.4) (layer "F.Cu") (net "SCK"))
 (segment (start 118.999 142.24) (end 119.698 142.938) (width 0.2) (layer "F.Cu") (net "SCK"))
 (segment (start 113.03 139.7) (end 114.3 138.43) (width 0.2) (layer "F.Cu") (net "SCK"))
 (segment (start 118.491 153.035) (end 119.698 151.828) (width 0.4) (layer "F.Cu") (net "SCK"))
 (segment (start 143.637 132.334) (end 145.415 134.112) (width 0.4) (layer "F.Cu") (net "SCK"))
 (segment (start 145.415 134.112) (end 145.415 134.62) (width 0.4) (layer "F.Cu") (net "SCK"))
 (segment (start 119.698 151.828) (end 119.698 142.938) (width 0.4) (layer "F.Cu") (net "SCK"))
 (segment (start 124.968 132.334) (end 143.637 132.334) (width 0.4) (layer "F.Cu") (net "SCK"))
 (segment (start 143.335744 133.096) (end 126.746 133.096) (width 0.4) (layer "F.Cu") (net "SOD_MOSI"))
 (segment (start 124.206 152.4) (end 124.841 151.765) (width 0.4) (layer "F.Cu") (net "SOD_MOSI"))
 (segment (start 125.095 155.575) (end 124.206 154.686) (width 0.4) (layer "F.Cu") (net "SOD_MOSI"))
 (segment (start 125.984 155.575) (end 125.095 155.575) (width 0.4) (layer "F.Cu") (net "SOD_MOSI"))
 (segment (start 131.826 140.97) (end 134.874 144.018) (width 0.4) (layer "F.Cu") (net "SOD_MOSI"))
 (segment (start 123.698 136.144) (end 123.698 139.7) (width 0.4) (layer "F.Cu") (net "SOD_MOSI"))
 (segment (start 143.335744 133.096) (end 144.145 133.905256) (width 0.2) (layer "F.Cu") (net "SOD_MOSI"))
 (segment (start 142.066 158.242) (end 139.399 155.575) (width 0.4) (layer "F.Cu") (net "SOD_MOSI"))
 (segment (start 141.605 135.89) (end 138.88 138.615) (width 0.2) (layer "F.Cu") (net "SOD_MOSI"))
 (segment (start 138.88 138.615) (end 138.88 140.335) (width 0.2) (layer "F.Cu") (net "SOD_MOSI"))
 (segment (start 132.969 151.765) (end 133.096 151.638) (width 0.4) (layer "F.Cu") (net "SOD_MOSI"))
 (segment (start 144.145 135.89) (end 141.605 135.89) (width 0.2) (layer "F.Cu") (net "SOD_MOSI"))
 (segment (start 126.746 133.096) (end 123.698 136.144) (width 0.4) (layer "F.Cu") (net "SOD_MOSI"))
 (segment (start 145.415 137.16) (end 144.145 135.89) (width 0.2) (layer "F.Cu") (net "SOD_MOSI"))
 (segment (start 128.27 140.97) (end 131.826 140.97) (width 0.4) (layer "F.Cu") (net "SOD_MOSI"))
 (segment (start 124.968 140.97) (end 125.956 140.97) (width 0.4) (layer "F.Cu") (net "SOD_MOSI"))
 (segment (start 124.206 154.686) (end 124.206 152.4) (width 0.4) (layer "F.Cu") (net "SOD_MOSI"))
 (segment (start 139.399 155.575) (end 128.27 155.575) (width 0.4) (layer "F.Cu") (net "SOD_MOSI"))
 (segment (start 134.874 149.86) (end 132.969 151.765) (width 0.4) (layer "F.Cu") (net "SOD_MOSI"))
 (segment (start 124.841 151.765) (end 132.969 151.765) (width 0.4) (layer "F.Cu") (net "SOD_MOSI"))
 (segment (start 134.874 144.018) (end 134.874 149.86) (width 0.4) (layer "F.Cu") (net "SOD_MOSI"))
 (segment (start 144.145 133.905256) (end 144.145 135.89) (width 0.2) (layer "F.Cu") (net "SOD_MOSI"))
 (segment (start 123.698 139.7) (end 124.968 140.97) (width 0.4) (layer "F.Cu") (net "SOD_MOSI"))
 (segment (start 140.97 134.62) (end 135.89 139.7) (width 0.4) (layer "F.Cu") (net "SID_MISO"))
 (segment (start 128.27 138.43) (end 133.985 138.43) (width 0.4) (layer "F.Cu") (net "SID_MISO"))
 (segment (start 142.875 134.62) (end 140.97 134.62) (width 0.4) (layer "F.Cu") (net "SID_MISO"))
 (segment (start 133.985 138.43) (end 135.89 140.335) (width 0.4) (layer "F.Cu") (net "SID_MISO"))
 (segment (start 135.89 153.035) (end 128.27 153.035) (width 0.4) (layer "F.Cu") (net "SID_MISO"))
 (segment (start 140.335 153.035) (end 135.89 153.035) (width 0.4) (layer "F.Cu") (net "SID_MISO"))
 (segment (start 144.566 158.242) (end 144.566 157.266) (width 0.4) (layer "F.Cu") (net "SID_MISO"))
 (segment (start 125.984 153.035) (end 127.635 153.035) (width 0.2) (layer "F.Cu") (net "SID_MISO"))
 (segment (start 135.89 140.335) (end 135.89 153.035) (width 0.4) (layer "F.Cu") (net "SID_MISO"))
 (segment (start 125.956 138.43) (end 127.635 138.43) (width 0.2) (layer "F.Cu") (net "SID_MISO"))
 (segment (start 135.89 139.7) (end 135.89 140.335) (width 0.4) (layer "F.Cu") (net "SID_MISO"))
 (segment (start 144.566 157.266) (end 140.335 153.035) (width 0.4) (layer "F.Cu") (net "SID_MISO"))
 (segment (start 144.78 144.78) (end 147.32 144.78) (width 0.4) (layer "F.Cu") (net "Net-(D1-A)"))
 (segment (start 149.566 158.242) (end 149.566 152.661) (width 1.27) (layer "F.Cu") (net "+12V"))
 (segment (start 142.326 145.421) (end 142.326 144.794) (width 1.27) (layer "F.Cu") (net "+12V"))
 (segment (start 149.566 152.661) (end 142.326 145.421) (width 1.27) (layer "F.Cu") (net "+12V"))
 (segment (start 139.7 144.78) (end 139.7 145.905) (width 0.4) (layer "F.Cu") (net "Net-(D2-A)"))
 (segment (start 139.7 145.905) (end 140.97 147.175) (width 0.4) (layer "F.Cu") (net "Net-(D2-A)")))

